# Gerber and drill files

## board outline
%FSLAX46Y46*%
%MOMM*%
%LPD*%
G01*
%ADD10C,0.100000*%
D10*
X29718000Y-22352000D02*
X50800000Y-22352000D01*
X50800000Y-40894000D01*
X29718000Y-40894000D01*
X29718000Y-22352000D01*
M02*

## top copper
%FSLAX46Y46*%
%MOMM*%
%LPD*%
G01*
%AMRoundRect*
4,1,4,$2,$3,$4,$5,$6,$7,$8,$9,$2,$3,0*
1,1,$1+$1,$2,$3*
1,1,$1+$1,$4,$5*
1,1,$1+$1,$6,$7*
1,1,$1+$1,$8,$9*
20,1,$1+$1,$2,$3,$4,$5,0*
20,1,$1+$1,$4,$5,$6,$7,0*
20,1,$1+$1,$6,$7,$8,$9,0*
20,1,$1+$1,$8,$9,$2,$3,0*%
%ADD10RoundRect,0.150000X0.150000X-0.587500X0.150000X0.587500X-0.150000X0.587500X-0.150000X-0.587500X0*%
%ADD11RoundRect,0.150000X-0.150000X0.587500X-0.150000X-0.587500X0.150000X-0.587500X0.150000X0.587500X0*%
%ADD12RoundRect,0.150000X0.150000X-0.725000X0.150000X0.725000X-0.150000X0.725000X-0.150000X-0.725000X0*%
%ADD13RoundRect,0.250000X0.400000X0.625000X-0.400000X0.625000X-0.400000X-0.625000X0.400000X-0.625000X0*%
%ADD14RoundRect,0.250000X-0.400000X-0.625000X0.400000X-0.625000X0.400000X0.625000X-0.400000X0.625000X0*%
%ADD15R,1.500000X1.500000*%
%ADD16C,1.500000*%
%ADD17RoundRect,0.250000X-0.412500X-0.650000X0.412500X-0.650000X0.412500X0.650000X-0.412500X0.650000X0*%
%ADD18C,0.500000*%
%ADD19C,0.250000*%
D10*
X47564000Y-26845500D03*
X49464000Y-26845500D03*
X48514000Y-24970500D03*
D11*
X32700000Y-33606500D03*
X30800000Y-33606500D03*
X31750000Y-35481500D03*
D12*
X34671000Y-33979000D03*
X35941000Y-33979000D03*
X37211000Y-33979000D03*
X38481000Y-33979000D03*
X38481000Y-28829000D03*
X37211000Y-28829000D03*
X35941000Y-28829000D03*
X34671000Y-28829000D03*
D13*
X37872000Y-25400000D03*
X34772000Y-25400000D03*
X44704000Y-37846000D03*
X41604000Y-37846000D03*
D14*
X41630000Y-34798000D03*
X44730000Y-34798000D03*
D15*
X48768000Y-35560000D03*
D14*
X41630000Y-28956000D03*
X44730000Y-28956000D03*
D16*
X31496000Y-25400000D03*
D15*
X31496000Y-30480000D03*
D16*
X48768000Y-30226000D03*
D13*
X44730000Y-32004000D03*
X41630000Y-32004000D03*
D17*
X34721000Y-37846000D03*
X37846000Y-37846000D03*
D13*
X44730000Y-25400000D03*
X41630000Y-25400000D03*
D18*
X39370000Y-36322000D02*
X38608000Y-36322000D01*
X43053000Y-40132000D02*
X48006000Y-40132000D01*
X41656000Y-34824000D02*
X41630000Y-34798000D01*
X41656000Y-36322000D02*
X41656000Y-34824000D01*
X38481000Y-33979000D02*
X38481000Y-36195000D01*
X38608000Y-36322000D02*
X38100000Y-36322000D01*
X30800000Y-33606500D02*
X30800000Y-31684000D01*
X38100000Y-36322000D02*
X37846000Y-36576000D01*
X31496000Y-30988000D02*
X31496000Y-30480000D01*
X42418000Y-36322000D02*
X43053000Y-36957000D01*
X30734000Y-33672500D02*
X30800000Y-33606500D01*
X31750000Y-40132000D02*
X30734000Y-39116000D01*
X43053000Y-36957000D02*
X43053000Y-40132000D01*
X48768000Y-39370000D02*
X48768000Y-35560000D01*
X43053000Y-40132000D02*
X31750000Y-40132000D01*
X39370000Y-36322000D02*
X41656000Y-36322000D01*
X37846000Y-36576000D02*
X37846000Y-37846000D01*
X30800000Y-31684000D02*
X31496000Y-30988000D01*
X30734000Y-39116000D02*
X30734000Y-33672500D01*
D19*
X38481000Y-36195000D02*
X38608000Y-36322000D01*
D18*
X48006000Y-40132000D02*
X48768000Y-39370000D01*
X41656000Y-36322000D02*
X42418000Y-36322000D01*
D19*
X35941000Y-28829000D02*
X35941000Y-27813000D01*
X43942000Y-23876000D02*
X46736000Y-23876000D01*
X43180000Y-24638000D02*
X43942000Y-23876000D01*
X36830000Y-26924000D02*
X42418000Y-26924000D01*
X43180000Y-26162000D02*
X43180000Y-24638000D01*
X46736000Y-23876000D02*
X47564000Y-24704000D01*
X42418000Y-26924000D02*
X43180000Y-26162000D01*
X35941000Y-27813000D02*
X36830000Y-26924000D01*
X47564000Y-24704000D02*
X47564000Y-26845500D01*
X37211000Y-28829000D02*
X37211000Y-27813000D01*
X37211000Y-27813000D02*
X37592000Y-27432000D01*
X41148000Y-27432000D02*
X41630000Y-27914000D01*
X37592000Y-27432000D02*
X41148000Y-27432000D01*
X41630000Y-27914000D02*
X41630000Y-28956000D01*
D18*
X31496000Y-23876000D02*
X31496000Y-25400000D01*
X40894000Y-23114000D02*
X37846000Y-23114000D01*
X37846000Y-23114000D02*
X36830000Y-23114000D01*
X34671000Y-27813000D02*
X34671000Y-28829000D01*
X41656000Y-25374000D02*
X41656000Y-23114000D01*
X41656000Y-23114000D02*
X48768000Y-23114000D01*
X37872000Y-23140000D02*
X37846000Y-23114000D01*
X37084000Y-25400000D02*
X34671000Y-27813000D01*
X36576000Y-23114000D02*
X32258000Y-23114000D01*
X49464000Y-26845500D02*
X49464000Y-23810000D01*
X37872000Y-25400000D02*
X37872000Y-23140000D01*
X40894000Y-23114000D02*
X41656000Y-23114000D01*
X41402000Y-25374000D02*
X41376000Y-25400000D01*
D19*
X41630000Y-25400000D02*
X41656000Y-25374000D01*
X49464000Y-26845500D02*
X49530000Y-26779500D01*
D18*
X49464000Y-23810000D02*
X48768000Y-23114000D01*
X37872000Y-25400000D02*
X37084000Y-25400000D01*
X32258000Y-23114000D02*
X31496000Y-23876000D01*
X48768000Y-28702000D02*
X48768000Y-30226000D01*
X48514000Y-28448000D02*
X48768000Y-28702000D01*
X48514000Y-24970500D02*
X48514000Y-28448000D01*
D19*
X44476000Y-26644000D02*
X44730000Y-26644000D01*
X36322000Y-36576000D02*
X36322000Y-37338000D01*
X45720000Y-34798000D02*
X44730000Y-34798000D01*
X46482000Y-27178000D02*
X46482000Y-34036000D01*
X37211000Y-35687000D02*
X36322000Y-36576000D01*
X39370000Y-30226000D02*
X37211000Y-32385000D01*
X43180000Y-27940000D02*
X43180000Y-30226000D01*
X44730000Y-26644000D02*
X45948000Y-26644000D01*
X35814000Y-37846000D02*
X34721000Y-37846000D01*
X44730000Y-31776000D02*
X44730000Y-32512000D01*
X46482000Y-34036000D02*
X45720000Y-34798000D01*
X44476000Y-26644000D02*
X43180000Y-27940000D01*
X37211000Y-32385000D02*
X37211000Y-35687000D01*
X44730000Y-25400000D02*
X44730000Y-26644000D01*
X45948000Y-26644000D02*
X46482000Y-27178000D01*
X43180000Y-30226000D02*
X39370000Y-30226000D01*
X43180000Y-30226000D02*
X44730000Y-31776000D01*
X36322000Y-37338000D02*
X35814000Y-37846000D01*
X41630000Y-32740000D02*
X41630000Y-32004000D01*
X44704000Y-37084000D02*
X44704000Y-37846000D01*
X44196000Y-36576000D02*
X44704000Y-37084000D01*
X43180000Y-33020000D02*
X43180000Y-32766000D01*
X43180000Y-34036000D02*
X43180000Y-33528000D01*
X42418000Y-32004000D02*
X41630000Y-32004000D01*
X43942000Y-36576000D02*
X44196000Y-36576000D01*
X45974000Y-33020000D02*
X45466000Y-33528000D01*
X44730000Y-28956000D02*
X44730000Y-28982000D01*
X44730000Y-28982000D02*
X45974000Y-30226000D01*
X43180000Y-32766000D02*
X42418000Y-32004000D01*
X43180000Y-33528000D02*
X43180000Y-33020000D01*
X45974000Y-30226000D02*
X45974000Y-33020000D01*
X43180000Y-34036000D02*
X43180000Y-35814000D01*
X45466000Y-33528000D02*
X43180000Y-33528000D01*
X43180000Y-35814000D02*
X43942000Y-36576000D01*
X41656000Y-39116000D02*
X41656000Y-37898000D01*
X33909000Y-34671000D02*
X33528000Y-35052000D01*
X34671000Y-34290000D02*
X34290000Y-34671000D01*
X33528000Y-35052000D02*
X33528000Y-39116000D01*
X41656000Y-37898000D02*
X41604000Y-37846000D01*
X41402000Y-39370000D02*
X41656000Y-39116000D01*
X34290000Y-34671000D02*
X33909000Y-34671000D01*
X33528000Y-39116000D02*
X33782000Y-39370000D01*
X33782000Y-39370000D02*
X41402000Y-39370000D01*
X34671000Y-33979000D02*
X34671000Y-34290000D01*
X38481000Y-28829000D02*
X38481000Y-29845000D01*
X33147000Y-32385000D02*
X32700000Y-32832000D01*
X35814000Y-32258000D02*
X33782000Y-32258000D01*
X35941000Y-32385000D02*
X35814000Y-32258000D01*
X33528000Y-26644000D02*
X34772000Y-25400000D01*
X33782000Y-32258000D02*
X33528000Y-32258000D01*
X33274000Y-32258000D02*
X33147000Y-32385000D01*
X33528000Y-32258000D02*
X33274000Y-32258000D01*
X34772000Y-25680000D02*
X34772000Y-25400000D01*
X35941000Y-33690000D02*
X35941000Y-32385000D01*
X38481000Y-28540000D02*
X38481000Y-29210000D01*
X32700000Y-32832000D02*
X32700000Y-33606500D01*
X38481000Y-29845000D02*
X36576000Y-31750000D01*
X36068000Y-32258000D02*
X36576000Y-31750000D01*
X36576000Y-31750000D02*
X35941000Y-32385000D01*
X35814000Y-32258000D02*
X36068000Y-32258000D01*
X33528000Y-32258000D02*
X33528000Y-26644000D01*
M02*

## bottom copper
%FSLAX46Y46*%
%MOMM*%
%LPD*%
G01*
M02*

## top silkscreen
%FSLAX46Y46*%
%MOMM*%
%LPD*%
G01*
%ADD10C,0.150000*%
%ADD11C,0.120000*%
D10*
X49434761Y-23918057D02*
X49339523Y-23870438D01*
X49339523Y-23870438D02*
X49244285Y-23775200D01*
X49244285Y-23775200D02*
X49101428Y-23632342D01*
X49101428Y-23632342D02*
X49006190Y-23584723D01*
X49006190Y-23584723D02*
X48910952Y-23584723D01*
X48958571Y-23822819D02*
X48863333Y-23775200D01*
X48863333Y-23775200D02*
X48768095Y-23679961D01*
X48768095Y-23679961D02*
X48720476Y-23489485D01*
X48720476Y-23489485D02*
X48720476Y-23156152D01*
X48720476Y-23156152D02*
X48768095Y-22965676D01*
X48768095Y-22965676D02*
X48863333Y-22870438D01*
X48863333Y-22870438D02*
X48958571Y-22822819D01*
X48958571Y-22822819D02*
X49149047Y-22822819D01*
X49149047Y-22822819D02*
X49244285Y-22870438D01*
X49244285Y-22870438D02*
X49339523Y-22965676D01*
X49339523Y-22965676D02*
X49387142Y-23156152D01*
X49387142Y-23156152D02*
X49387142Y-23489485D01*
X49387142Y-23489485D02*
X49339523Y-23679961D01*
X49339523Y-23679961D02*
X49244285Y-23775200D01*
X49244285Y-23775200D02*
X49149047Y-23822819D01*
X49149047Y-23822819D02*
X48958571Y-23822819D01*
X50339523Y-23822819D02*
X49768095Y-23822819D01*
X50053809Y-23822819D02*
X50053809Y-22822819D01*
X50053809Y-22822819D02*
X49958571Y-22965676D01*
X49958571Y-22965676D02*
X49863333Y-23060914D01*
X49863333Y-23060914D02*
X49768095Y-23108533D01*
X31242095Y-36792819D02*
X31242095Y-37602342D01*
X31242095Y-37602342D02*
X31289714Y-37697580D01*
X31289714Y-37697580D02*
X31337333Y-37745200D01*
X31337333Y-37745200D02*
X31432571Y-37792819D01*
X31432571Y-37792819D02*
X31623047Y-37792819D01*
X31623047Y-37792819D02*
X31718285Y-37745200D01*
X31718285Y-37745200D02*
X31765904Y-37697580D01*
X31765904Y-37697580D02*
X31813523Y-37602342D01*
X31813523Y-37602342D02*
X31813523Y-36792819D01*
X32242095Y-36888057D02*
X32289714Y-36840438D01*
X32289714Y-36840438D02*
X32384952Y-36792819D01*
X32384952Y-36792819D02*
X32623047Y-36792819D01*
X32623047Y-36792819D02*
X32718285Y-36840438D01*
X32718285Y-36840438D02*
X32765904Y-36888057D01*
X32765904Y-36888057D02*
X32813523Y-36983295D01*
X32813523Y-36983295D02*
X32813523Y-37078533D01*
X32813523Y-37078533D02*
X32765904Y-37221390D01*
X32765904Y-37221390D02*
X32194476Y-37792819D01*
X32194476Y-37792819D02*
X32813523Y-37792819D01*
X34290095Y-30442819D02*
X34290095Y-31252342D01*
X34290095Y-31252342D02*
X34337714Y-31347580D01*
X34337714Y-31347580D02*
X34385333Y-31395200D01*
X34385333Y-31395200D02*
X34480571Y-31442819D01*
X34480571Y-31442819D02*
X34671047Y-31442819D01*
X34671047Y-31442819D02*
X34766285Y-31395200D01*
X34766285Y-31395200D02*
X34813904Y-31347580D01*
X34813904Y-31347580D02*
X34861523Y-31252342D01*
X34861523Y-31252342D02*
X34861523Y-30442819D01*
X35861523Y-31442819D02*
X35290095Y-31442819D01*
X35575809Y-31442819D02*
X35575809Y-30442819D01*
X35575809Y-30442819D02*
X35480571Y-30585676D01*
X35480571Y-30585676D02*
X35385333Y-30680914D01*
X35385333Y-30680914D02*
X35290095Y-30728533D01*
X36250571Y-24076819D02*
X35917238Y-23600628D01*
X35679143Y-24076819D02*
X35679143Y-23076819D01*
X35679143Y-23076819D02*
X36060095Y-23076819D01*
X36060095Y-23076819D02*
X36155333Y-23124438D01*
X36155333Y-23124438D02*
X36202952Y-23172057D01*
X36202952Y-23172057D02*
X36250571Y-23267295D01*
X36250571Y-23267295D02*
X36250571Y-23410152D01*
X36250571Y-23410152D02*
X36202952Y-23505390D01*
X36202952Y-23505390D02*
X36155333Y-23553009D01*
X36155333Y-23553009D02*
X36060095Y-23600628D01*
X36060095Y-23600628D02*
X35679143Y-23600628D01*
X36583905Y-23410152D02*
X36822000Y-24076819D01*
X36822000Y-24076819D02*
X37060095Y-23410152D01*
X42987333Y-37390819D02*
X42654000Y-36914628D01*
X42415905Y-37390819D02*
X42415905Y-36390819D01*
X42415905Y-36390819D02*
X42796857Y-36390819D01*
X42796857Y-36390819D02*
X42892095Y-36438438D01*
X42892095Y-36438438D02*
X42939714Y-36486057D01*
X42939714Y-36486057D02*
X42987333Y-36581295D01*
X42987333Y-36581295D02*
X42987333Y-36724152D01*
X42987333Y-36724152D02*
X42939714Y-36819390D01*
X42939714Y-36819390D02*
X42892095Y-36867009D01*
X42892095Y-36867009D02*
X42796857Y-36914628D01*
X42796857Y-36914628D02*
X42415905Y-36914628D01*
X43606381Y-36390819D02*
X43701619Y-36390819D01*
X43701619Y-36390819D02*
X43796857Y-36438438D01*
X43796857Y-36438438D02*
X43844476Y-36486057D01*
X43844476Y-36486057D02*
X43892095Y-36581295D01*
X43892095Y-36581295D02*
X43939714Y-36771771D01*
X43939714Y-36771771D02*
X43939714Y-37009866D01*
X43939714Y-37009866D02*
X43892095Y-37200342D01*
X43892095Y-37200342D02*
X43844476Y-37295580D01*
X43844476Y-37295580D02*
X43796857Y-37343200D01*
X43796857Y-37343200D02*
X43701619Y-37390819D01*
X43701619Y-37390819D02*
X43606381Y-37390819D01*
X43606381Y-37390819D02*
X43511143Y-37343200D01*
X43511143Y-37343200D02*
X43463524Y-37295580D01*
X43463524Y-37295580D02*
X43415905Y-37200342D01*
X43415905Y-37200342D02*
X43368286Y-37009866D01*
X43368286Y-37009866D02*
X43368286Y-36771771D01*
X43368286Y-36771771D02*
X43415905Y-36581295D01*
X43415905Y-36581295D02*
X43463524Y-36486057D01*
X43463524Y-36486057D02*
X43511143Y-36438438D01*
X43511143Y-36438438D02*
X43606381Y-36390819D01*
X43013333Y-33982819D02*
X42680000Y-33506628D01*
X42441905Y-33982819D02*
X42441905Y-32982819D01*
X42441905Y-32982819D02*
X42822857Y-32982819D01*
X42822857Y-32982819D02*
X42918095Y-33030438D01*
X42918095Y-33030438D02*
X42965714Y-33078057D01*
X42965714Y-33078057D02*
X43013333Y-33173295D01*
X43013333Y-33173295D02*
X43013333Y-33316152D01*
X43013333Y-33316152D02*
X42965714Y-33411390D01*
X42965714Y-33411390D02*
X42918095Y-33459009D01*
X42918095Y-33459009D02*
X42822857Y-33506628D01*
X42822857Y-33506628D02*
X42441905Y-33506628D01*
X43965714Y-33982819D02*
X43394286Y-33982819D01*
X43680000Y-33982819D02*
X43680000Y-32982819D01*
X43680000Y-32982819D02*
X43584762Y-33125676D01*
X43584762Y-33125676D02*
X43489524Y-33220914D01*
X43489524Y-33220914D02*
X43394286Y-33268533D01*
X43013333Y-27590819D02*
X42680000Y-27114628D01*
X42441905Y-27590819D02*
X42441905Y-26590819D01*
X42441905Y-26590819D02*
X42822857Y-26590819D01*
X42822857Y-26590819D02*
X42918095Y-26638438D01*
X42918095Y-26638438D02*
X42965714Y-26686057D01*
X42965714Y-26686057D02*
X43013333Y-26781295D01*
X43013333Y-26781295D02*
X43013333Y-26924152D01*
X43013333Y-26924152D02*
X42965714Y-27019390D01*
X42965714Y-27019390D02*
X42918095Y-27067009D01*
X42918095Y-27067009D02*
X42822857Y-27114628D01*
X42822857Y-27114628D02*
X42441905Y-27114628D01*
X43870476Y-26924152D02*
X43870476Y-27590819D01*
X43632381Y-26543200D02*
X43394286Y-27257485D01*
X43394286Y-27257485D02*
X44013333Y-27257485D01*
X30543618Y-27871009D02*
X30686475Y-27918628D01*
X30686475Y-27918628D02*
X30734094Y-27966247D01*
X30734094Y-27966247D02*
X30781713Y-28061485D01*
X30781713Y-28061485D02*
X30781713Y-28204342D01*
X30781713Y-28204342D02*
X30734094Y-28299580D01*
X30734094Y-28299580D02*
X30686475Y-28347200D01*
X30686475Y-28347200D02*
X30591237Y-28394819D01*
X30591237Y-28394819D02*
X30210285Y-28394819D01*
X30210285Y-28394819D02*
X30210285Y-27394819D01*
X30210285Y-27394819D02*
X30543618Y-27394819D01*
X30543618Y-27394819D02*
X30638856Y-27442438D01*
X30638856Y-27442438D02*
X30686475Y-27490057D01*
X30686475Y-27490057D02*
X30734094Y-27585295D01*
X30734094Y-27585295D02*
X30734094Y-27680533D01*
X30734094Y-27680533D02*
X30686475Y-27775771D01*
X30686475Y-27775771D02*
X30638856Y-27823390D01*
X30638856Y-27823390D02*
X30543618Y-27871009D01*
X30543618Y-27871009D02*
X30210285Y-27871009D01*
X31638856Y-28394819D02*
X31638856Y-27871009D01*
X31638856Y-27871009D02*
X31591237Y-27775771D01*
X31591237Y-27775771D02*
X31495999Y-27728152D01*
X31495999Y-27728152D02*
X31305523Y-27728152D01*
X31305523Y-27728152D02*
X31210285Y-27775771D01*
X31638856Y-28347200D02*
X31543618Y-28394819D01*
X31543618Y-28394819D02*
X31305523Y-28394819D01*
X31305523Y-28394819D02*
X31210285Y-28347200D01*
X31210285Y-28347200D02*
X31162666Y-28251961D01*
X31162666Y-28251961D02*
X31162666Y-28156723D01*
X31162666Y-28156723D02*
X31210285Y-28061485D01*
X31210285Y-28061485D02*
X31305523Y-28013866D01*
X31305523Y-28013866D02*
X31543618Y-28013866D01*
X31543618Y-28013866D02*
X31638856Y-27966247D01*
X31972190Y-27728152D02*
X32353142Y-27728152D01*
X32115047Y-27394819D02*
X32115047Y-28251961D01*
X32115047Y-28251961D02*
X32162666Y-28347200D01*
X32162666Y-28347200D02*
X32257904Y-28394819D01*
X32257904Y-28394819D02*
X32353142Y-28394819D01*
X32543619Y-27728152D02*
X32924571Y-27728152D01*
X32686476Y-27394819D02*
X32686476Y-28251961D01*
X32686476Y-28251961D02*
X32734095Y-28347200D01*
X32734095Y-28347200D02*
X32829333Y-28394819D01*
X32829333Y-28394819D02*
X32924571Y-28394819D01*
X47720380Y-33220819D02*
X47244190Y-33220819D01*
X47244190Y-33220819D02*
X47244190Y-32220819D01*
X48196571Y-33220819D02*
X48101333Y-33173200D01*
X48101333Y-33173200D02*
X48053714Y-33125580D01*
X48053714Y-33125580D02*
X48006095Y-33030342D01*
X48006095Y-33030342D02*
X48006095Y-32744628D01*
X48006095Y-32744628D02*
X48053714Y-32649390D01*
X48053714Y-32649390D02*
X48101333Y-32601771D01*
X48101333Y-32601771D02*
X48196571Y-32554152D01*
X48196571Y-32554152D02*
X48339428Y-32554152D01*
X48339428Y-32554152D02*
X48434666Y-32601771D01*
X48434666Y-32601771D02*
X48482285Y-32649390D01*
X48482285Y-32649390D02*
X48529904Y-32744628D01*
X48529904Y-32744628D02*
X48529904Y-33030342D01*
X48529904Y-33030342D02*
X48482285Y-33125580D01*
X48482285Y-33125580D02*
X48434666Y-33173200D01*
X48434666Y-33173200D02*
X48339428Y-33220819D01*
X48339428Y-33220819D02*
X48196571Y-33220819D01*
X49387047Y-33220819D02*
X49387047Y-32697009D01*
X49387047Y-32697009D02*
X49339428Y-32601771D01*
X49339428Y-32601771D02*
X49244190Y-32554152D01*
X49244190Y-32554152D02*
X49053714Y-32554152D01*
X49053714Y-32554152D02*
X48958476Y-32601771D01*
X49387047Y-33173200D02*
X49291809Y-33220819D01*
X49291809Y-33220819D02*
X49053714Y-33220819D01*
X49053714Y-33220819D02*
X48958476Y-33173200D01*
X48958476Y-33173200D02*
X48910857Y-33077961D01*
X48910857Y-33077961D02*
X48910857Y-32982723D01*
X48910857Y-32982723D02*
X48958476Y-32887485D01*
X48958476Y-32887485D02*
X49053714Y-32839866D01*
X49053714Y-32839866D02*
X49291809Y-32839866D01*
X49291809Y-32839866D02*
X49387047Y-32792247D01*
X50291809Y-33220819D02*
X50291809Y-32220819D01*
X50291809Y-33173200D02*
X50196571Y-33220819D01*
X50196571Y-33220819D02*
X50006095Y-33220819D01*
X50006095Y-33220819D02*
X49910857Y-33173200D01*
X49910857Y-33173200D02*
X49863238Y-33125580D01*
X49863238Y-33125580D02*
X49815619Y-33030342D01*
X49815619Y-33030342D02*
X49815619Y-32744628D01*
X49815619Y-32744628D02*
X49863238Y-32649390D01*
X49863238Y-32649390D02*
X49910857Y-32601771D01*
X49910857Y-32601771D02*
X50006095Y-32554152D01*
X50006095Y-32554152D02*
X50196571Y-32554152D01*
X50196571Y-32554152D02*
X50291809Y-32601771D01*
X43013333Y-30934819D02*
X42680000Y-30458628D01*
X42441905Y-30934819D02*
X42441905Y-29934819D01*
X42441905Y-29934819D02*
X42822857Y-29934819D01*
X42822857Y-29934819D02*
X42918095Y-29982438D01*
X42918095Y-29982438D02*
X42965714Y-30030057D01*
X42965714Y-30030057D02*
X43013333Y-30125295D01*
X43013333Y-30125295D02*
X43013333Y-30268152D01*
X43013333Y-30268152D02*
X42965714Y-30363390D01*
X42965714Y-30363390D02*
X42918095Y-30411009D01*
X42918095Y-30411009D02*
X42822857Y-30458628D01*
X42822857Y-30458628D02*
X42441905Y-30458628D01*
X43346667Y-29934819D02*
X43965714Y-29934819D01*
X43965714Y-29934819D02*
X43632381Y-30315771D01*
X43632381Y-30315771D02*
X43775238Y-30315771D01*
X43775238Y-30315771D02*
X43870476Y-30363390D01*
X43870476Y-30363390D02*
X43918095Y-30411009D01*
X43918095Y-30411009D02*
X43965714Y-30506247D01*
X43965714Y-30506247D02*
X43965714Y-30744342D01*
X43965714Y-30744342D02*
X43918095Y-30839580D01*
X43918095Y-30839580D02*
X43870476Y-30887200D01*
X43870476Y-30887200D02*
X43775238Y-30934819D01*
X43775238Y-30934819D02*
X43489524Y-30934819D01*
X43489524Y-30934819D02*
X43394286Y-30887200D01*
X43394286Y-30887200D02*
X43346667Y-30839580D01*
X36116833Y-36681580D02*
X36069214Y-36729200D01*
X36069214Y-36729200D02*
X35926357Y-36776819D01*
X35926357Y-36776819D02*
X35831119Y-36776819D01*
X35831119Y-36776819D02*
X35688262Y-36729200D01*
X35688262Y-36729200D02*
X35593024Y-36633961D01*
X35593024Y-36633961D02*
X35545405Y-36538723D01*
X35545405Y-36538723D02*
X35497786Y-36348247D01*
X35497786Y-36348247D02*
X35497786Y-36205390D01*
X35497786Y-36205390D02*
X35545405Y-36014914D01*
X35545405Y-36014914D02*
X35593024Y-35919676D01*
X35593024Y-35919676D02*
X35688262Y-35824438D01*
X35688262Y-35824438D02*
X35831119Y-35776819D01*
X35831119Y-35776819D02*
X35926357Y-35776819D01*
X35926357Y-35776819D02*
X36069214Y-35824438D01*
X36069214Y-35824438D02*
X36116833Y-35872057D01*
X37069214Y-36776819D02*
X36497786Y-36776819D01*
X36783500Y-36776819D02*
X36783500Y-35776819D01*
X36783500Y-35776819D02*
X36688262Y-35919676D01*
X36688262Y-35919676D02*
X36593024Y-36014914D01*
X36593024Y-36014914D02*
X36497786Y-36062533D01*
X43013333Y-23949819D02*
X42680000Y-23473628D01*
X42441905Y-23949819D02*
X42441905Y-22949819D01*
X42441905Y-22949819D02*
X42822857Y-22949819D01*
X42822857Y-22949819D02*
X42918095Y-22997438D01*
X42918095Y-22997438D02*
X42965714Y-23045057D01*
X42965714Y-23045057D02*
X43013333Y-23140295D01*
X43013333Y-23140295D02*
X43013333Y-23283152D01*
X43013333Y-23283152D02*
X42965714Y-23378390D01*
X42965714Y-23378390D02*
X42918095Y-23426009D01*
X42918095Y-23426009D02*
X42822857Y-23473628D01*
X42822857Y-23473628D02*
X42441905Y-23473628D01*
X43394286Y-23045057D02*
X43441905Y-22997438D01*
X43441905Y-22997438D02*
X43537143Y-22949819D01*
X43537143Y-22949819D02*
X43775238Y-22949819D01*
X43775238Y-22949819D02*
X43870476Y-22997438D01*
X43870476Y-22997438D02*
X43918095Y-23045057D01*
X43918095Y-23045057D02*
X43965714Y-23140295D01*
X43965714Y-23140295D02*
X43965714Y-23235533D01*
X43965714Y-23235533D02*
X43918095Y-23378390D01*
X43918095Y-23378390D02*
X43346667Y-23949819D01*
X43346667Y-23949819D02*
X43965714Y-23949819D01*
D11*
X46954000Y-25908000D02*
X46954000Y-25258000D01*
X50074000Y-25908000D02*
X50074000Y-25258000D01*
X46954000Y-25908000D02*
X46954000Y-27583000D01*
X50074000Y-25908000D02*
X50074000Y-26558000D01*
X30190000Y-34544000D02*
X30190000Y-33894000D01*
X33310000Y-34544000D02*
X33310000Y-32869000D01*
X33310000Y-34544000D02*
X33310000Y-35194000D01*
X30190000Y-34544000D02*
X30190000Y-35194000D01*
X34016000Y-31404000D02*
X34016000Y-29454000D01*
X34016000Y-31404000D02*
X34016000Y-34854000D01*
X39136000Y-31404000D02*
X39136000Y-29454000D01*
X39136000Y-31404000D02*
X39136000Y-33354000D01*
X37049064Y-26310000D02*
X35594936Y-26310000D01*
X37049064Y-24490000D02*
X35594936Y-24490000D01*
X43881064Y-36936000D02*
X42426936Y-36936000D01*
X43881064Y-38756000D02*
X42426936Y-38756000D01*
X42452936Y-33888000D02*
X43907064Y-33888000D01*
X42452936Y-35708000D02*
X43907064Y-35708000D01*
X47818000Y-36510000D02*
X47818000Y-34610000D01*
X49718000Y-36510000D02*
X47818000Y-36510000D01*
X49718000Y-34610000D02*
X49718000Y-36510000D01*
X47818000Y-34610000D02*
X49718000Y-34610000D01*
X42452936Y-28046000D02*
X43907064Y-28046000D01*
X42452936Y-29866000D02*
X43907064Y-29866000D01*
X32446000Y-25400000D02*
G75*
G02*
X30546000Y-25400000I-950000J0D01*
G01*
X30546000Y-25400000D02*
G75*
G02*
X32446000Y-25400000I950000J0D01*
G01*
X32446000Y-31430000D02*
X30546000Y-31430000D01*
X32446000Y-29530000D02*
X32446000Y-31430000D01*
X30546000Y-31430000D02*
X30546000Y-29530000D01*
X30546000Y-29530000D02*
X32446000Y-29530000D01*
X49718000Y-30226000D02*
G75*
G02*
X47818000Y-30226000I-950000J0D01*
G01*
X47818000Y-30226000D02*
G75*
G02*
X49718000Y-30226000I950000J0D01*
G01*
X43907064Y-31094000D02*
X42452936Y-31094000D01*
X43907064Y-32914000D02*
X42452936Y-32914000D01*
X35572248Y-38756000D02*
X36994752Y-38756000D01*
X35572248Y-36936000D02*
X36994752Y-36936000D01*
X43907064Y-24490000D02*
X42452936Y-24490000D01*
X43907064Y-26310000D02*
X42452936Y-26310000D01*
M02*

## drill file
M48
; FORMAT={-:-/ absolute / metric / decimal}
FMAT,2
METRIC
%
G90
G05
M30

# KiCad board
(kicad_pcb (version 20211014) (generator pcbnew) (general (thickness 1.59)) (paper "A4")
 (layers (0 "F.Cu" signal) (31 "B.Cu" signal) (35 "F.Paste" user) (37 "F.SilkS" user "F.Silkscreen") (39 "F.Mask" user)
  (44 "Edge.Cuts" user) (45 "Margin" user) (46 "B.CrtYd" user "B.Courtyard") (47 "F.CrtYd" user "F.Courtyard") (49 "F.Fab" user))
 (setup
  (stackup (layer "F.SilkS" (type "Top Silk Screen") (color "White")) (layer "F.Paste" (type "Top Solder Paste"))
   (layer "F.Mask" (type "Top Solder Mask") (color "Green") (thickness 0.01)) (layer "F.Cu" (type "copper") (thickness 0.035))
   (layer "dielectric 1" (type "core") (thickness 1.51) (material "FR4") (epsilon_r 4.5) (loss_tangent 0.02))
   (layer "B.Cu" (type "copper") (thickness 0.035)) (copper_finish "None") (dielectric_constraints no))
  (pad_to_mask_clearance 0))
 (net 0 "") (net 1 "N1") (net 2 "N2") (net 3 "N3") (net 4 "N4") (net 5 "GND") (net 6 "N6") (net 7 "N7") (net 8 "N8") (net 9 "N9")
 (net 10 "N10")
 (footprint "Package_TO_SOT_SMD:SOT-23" (layer "F.Cu") (at 48.514 25.908 90)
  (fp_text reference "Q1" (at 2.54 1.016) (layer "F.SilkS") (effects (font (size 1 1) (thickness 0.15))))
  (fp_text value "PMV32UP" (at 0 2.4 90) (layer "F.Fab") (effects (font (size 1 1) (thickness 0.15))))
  (fp_line (start 0 -1.56) (end 0.65 -1.56) (layer "F.SilkS") (width 0.12))
  (fp_line (start 0 1.56) (end 0.65 1.56) (layer "F.SilkS") (width 0.12))
  (fp_line (start 0 -1.56) (end -1.675 -1.56) (layer "F.SilkS") (width 0.12))
  (fp_line (start 0 1.56) (end -0.65 1.56) (layer "F.SilkS") (width 0.12))
  (pad "1" smd roundrect (at -0.9375 -0.95 90) (size 1.475 0.6) (layers "F.Cu" "F.Paste" "F.Mask") (roundrect_rratio 0.25) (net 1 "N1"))
  (pad "2" smd roundrect (at -0.9375 0.95 90) (size 1.475 0.6) (layers "F.Cu" "F.Paste" "F.Mask") (roundrect_rratio 0.25) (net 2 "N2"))
  (pad "3" smd roundrect (at 0.9375 0 90) (size 1.475 0.6) (layers "F.Cu" "F.Paste" "F.Mask") (roundrect_rratio 0.25) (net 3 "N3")))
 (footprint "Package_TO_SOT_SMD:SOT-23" (layer "F.Cu") (at 31.75 34.544 -90)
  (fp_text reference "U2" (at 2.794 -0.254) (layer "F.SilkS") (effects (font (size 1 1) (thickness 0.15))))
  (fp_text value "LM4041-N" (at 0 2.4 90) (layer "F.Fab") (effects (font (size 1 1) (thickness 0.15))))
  (fp_line (start 0 1.56) (end -0.65 1.56) (layer "F.SilkS") (width 0.12))
  (fp_line (start 0 -1.56) (end -1.675 -1.56) (layer "F.SilkS") (width 0.12))
  (fp_line (start 0 -1.56) (end 0.65 -1.56) (layer "F.SilkS") (width 0.12))
  (fp_line (start 0 1.56) (end 0.65 1.56) (layer "F.SilkS") (width 0.12))
  (pad "1" smd roundrect (at -0.9375 -0.95 270) (size 1.475 0.6) (layers "F.Cu" "F.Paste" "F.Mask") (roundrect_rratio 0.25) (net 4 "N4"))
  (pad "2" smd roundrect (at -0.9375 0.95 270) (size 1.475 0.6) (layers "F.Cu" "F.Paste" "F.Mask") (roundrect_rratio 0.25) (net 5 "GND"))
  (pad "3" smd roundrect (at 0.9375 0 270) (size 1.475 0.6) (layers "F.Cu" "F.Paste" "F.Mask") (roundrect_rratio 0.25) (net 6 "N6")))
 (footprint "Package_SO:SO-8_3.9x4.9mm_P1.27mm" (layer "F.Cu") (at 36.576 31.404 90)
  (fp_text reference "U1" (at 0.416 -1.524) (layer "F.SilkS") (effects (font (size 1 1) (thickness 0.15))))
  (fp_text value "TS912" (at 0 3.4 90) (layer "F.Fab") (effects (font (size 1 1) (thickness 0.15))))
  (fp_line (start 0 -2.56) (end 1.95 -2.56) (layer "F.SilkS") (width 0.12))
  (fp_line (start 0 -2.56) (end -3.45 -2.56) (layer "F.SilkS") (width 0.12))
  (fp_line (start 0 2.56) (end 1.95 2.56) (layer "F.SilkS") (width 0.12))
  (fp_line (start 0 2.56) (end -1.95 2.56) (layer "F.SilkS") (width 0.12))
  (pad "1" smd roundrect (at -2.575 -1.905 90) (size 1.75 0.6) (layers "F.Cu" "F.Paste" "F.Mask") (roundrect_rratio 0.25) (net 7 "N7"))
  (pad "2" smd roundrect (at -2.575 -0.635 90) (size 1.75 0.6) (layers "F.Cu" "F.Paste" "F.Mask") (roundrect_rratio 0.25) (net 4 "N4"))
  (pad "3" smd roundrect (at -2.575 0.635 90) (size 1.75 0.6) (layers "F.Cu" "F.Paste" "F.Mask") (roundrect_rratio 0.25) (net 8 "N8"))
  (pad "4" smd roundrect (at -2.575 1.905 90) (size 1.75 0.6) (layers "F.Cu" "F.Paste" "F.Mask") (roundrect_rratio 0.25) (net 5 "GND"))
  (pad "5" smd roundrect (at 2.575 1.905 90) (size 1.75 0.6) (layers "F.Cu" "F.Paste" "F.Mask") (roundrect_rratio 0.25) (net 4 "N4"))
  (pad "6" smd roundrect (at 2.575 0.635 90) (size 1.75 0.6) (layers "F.Cu" "F.Paste" "F.Mask") (roundrect_rratio 0.25) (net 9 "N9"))
  (pad "7" smd roundrect (at 2.575 -0.635 90) (size 1.75 0.6) (layers "F.Cu" "F.Paste" "F.Mask") (roundrect_rratio 0.25) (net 1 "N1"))
  (pad "8" smd roundrect (at 2.575 -1.905 90) (size 1.75 0.6) (layers "F.Cu" "F.Paste" "F.Mask") (roundrect_rratio 0.25) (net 2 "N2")))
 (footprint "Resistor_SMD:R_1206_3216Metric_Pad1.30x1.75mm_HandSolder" (layer "F.Cu") (at 36.322 25.4 180)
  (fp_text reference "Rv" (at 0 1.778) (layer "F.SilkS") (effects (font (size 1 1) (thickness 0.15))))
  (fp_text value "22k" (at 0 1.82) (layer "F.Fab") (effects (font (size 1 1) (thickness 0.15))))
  (fp_line (start -0.727064 -0.91) (end 0.727064 -0.91) (layer "F.SilkS") (width 0.12))
  (fp_line (start -0.727064 0.91) (end 0.727064 0.91) (layer "F.SilkS") (width 0.12))
  (pad "1" smd roundrect (at -1.55 0 180) (size 1.3 1.75) (layers "F.Cu" "F.Paste" "F.Mask") (roundrect_rratio 0.1923076923) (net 2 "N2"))
  (pad "2" smd roundrect (at 1.55 0 180) (size 1.3 1.75) (layers "F.Cu" "F.Paste" "F.Mask") (roundrect_rratio 0.1923076923) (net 4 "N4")))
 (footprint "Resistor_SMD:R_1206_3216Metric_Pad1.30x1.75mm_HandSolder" (layer "F.Cu") (at 43.154 37.846 180)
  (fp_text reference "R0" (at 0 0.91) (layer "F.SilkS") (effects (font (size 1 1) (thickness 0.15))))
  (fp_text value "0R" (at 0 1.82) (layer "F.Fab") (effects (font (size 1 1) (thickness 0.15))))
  (fp_line (start -0.727064 0.91) (end 0.727064 0.91) (layer "F.SilkS") (width 0.12))
  (fp_line (start -0.727064 -0.91) (end 0.727064 -0.91) (layer "F.SilkS") (width 0.12))
  (pad "1" smd roundrect (at -1.55 0 180) (size 1.3 1.75) (layers "F.Cu" "F.Paste" "F.Mask") (roundrect_rratio 0.192308) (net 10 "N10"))
  (pad "2" smd roundrect (at 1.55 0 180) (size 1.3 1.75) (layers "F.Cu" "F.Paste" "F.Mask") (roundrect_rratio 0.192308) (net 7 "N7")))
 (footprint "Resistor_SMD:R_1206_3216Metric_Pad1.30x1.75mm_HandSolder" (layer "F.Cu") (at 43.18 34.798)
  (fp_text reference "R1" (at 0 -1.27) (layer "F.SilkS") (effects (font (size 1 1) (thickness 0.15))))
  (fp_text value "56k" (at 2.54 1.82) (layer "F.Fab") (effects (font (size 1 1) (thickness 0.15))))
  (fp_line (start -0.727064 -0.91) (end 0.727064 -0.91) (layer "F.SilkS") (width 0.12))
  (fp_line (start -0.727064 0.91) (end 0.727064 0.91) (layer "F.SilkS") (width 0.12))
  (pad "1" smd roundrect (at -1.55 0) (size 1.3 1.75) (layers "F.Cu" "F.Paste" "F.Mask") (roundrect_rratio 0.1923076923) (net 5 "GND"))
  (pad "2" smd roundrect (at 1.55 0) (size 1.3 1.75) (layers "F.Cu" "F.Paste" "F.Mask") (roundrect_rratio 0.1923076923) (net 8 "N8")))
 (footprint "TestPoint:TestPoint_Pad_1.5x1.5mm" (layer "F.Cu") (at 48.768 35.56)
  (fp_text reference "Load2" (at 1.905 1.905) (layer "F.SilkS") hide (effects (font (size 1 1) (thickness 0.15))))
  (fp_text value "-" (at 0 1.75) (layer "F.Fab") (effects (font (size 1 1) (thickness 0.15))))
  (fp_line (start -0.95 0.95) (end -0.95 -0.95) (layer "F.SilkS") (width 0.12))
  (fp_line (start 0.95 0.95) (end -0.95 0.95) (layer "F.SilkS") (width 0.12))
  (fp_line (start 0.95 -0.95) (end 0.95 0.95) (layer "F.SilkS") (width 0.12))
  (fp_line (start -0.95 -0.95) (end 0.95 -0.95) (layer "F.SilkS") (width 0.12))
  (pad "1" smd rect (at 0 0) (size 1.5 1.5) (layers "F.Cu" "F.Mask") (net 5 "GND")))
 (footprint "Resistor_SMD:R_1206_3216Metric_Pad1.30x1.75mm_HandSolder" (layer "F.Cu") (at 43.18 28.956)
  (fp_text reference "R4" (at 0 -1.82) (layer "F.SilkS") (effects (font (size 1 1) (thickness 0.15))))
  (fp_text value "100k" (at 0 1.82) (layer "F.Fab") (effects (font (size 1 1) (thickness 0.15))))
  (fp_line (start -0.727064 -0.91) (end 0.727064 -0.91) (layer "F.SilkS") (width 0.12))
  (fp_line (start -0.727064 0.91) (end 0.727064 0.91) (layer "F.SilkS") (width 0.12))
  (pad "1" smd roundrect (at -1.55 0) (size 1.3 1.75) (layers "F.Cu" "F.Paste" "F.Mask") (roundrect_rratio 0.1923076923) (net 9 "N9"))
  (pad "2" smd roundrect (at 1.55 0) (size 1.3 1.75) (layers "F.Cu" "F.Paste" "F.Mask") (roundrect_rratio 0.1923076923) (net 10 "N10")))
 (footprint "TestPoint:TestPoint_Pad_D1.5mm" (layer "F.Cu") (at 31.496 25.4)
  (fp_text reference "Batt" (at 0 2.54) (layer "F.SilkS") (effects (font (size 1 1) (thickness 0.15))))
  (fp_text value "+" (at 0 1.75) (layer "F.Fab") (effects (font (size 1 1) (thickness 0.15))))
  (fp_circle (center 0 0) (end 0 0.95) (layer "F.SilkS") (width 0.12) (fill none))
  (pad "1" smd circle (at 0 0) (size 1.5 1.5) (layers "F.Cu" "F.Mask") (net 2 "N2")))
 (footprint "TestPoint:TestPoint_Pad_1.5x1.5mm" (layer "F.Cu") (at 31.496 30.48)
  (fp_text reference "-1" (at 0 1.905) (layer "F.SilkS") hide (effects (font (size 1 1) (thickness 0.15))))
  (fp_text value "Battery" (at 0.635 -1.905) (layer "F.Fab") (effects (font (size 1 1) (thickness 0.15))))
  (fp_line (start 0.95 0.95) (end -0.95 0.95) (layer "F.SilkS") (width 0.12))
  (fp_line (start 0.95 -0.95) (end 0.95 0.95) (layer "F.SilkS") (width 0.12))
  (fp_line (start -0.95 0.95) (end -0.95 -0.95) (layer "F.SilkS") (width 0.12))
  (fp_line (start -0.95 -0.95) (end 0.95 -0.95) (layer "F.SilkS") (width 0.12))
  (pad "1" smd rect (at 0 0) (size 1.5 1.5) (layers "F.Cu" "F.Mask") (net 5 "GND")))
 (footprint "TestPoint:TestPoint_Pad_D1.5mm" (layer "F.Cu") (at 48.768 30.226)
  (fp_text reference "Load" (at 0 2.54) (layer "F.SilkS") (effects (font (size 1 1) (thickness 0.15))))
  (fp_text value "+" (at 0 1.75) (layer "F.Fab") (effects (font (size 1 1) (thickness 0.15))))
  (fp_circle (center 0 0) (end 0 0.95) (layer "F.SilkS") (width 0.12) (fill none))
  (pad "1" smd circle (at 0 0) (size 1.5 1.5) (layers "F.Cu" "F.Mask") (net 3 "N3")))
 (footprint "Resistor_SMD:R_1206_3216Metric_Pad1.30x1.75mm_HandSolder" (layer "F.Cu") (at 43.18 32.004 180)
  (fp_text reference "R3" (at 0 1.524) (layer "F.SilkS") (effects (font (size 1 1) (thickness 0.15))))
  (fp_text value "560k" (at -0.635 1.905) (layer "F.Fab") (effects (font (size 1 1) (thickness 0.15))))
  (fp_line (start -0.727064 0.91) (end 0.727064 0.91) (layer "F.SilkS") (width 0.12))
  (fp_line (start -0.727064 -0.91) (end 0.727064 -0.91) (layer "F.SilkS") (width 0.12))
  (pad "1" smd roundrect (at -1.55 0 180) (size 1.3 1.75) (layers "F.Cu" "F.Paste" "F.Mask") (roundrect_rratio 0.1923076923) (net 8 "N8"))
  (pad "2" smd roundrect (at 1.55 0 180) (size 1.3 1.75) (layers "F.Cu" "F.Paste" "F.Mask") (roundrect_rratio 0.1923076923) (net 10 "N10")))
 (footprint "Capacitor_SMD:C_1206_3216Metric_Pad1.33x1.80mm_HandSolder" (layer "F.Cu") (at 36.2835 37.846)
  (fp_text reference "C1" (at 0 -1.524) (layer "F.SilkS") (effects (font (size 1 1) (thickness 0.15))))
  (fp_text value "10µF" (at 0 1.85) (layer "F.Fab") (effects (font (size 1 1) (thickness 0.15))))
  (fp_line (start -0.711252 0.91) (end 0.711252 0.91) (layer "F.SilkS") (width 0.12))
  (fp_line (start -0.711252 -0.91) (end 0.711252 -0.91) (layer "F.SilkS") (width 0.12))
  (pad "1" smd roundrect (at -1.5625 0) (size 1.325 1.8) (layers "F.Cu" "F.Paste" "F.Mask") (roundrect_rratio 0.1886792453) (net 8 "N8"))
  (pad "2" smd roundrect (at 1.5625 0) (size 1.325 1.8) (layers "F.Cu" "F.Paste" "F.Mask") (roundrect_rratio 0.1886792453) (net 5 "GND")))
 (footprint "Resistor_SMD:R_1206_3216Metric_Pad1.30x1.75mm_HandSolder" (layer "F.Cu") (at 43.18 25.4 180)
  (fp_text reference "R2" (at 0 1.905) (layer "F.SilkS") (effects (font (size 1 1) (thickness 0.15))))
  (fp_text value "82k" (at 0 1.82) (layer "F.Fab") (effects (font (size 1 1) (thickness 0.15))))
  (fp_line (start -0.727064 0.91) (end 0.727064 0.91) (layer "F.SilkS") (width 0.12))
  (fp_line (start -0.727064 -0.91) (end 0.727064 -0.91) (layer "F.SilkS") (width 0.12))
  (pad "1" smd roundrect (at -1.55 0 180) (size 1.3 1.75) (layers "F.Cu" "F.Paste" "F.Mask") (roundrect_rratio 0.1923076923) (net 8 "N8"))
  (pad "2" smd roundrect (at 1.55 0 180) (size 1.3 1.75) (layers "F.Cu" "F.Paste" "F.Mask") (roundrect_rratio 0.1923076923) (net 2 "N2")))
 (gr_rect (start 29.718 22.352) (end 50.8 40.894) (layer "Edge.Cuts") (width 0.1) (fill none))
 (segment (start 39.37 36.322) (end 38.608 36.322) (width 0.5) (layer "F.Cu") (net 5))
 (segment (start 43.053 40.132) (end 48.006 40.132) (width 0.5) (layer "F.Cu") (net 5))
 (segment (start 41.656 34.824) (end 41.63 34.798) (width 0.5) (layer "F.Cu") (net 5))
 (segment (start 41.656 36.322) (end 41.656 34.824) (width 0.5) (layer "F.Cu") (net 5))
 (segment (start 38.481 33.979) (end 38.481 36.195) (width 0.5) (layer "F.Cu") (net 5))
 (segment (start 38.608 36.322) (end 38.1 36.322) (width 0.5) (layer "F.Cu") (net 5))
 (segment (start 30.8 33.6065) (end 30.8 31.684) (width 0.5) (layer "F.Cu") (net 5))
 (segment (start 38.1 36.322) (end 37.846 36.576) (width 0.5) (layer "F.Cu") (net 5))
 (segment (start 31.496 30.988) (end 31.496 30.48) (width 0.5) (layer "F.Cu") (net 5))
 (segment (start 42.418 36.322) (end 43.053 36.957) (width 0.5) (layer "F.Cu") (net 5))
 (segment (start 30.734 33.6725) (end 30.8 33.6065) (width 0.5) (layer "F.Cu") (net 5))
 (segment (start 31.75 40.132) (end 30.734 39.116) (width 0.5) (layer "F.Cu") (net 5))
 (segment (start 43.053 36.957) (end 43.053 40.132) (width 0.5) (layer "F.Cu") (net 5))
 (segment (start 48.768 39.37) (end 48.768 35.56) (width 0.5) (layer "F.Cu") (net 5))
 (segment (start 43.053 40.132) (end 31.75 40.132) (width 0.5) (layer "F.Cu") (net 5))
 (segment (start 39.37 36.322) (end 41.656 36.322) (width 0.5) (layer "F.Cu") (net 5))
 (segment (start 37.846 36.576) (end 37.846 37.846) (width 0.5) (layer "F.Cu") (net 5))
 (segment (start 30.8 31.684) (end 31.496 30.988) (width 0.5) (layer "F.Cu") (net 5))
 (segment (start 30.734 39.116) (end 30.734 33.6725) (width 0.5) (layer "F.Cu") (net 5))
 (segment (start 38.481 36.195) (end 38.608 36.322) (width 0.25) (layer "F.Cu") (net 5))
 (segment (start 48.006 40.132) (end 48.768 39.37) (width 0.5) (layer "F.Cu") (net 5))
 (segment (start 41.656 36.322) (end 42.418 36.322) (width 0.5) (layer "F.Cu") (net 5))
 (segment (start 35.941 28.829) (end 35.941 27.813) (width 0.25) (layer "F.Cu") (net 1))
 (segment (start 43.942 23.876) (end 46.736 23.876) (width 0.25) (layer "F.Cu") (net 1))
 (segment (start 43.18 24.638) (end 43.942 23.876) (width 0.25) (layer "F.Cu") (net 1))
 (segment (start 36.83 26.924) (end 42.418 26.924) (width 0.25) (layer "F.Cu") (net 1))
 (segment (start 43.18 26.162) (end 43.18 24.638) (width 0.25) (layer "F.Cu") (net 1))
 (segment (start 46.736 23.876) (end 47.564 24.704) (width 0.25) (layer "F.Cu") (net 1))
 (segment (start 42.418 26.924) (end 43.18 26.162) (width 0.25) (layer "F.Cu") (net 1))
 (segment (start 35.941 27.813) (end 36.83 26.924) (width 0.25) (layer "F.Cu") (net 1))
 (segment (start 47.564 24.704) (end 47.564 26.8455) (width 0.25) (layer "F.Cu") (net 1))
 (segment (start 37.211 28.829) (end 37.211 27.813) (width 0.25) (layer "F.Cu") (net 9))
 (segment (start 37.211 27.813) (end 37.592 27.432) (width 0.25) (layer "F.Cu") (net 9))
 (segment (start 41.148 27.432) (end 41.63 27.914) (width 0.25) (layer "F.Cu") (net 9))
 (segment (start 37.592 27.432) (end 41.148 27.432) (width 0.25) (layer "F.Cu") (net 9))
 (segment (start 41.63 27.914) (end 41.63 28.956) (width 0.25) (layer "F.Cu") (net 9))
 (segment (start 31.496 23.876) (end 31.496 25.4) (width 0.5) (layer "F.Cu") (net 2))
 (segment (start 40.894 23.114) (end 37.846 23.114) (width 0.5) (layer "F.Cu") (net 2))
 (segment (start 37.846 23.114) (end 36.83 23.114) (width 0.5) (layer "F.Cu") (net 2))
 (segment (start 34.671 27.813) (end 34.671 28.829) (width 0.5) (layer "F.Cu") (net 2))
 (segment (start 41.656 25.374) (end 41.656 23.114) (width 0.5) (layer "F.Cu") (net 2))
 (segment (start 41.656 23.114) (end 48.768 23.114) (width 0.5) (layer "F.Cu") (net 2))
 (segment (start 37.872 23.14) (end 37.846 23.114) (width 0.5) (layer "F.Cu") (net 2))
 (segment (start 37.084 25.4) (end 34.671 27.813) (width 0.5) (layer "F.Cu") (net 2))
 (segment (start 36.576 23.114) (end 32.258 23.114) (width 0.5) (layer "F.Cu") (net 2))
 (segment (start 49.464 26.8455) (end 49.464 23.81) (width 0.5) (layer "F.Cu") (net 2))
 (segment (start 37.872 25.4) (end 37.872 23.14) (width 0.5) (layer "F.Cu") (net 2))
 (segment (start 40.894 23.114) (end 41.656 23.114) (width 0.5) (layer "F.Cu") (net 2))
 (segment (start 41.402 25.374) (end 41.376 25.4) (width 0.5) (layer "F.Cu") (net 2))
 (segment (start 41.63 25.4) (end 41.656 25.374) (width 0.25) (layer "F.Cu") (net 2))
 (segment (start 49.464 26.8455) (end 49.53 26.7795) (width 0.25) (layer "F.Cu") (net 2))
 (segment (start 49.464 23.81) (end 48.768 23.114) (width 0.5) (layer "F.Cu") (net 2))
 (segment (start 37.872 25.4) (end 37.084 25.4) (width 0.5) (layer "F.Cu") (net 2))
 (segment (start 32.258 23.114) (end 31.496 23.876) (width 0.5) (layer "F.Cu") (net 2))
 (segment (start 48.768 28.702) (end 48.768 30.226) (width 0.5) (layer "F.Cu") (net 3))
 (segment (start 48.514 28.448) (end 48.768 28.702) (width 0.5) (layer "F.Cu") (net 3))
 (segment (start 48.514 24.9705) (end 48.514 28.448) (width 0.5) (layer "F.Cu") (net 3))
 (segment (start 44.476 26.644) (end 44.73 26.644) (width 0.25) (layer "F.Cu") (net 8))
 (segment (start 36.322 36.576) (end 36.322 37.338) (width 0.25) (layer "F.Cu") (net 8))
 (segment (start 45.72 34.798) (end 44.73 34.798) (width 0.25) (layer "F.Cu") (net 8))
 (segment (start 46.482 27.178) (end 46.482 34.036) (width 0.25) (layer "F.Cu") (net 8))
 (segment (start 37.211 35.687) (end 36.322 36.576) (width 0.25) (layer "F.Cu") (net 8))
 (segment (start 39.37 30.226) (end 37.211 32.385) (width 0.25) (layer "F.Cu") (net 8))
 (segment (start 43.18 27.94) (end 43.18 30.226) (width 0.25) (layer "F.Cu") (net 8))
 (segment (start 44.73 26.644) (end 45.948 26.644) (width 0.25) (layer "F.Cu") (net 8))
 (segment (start 35.814 37.846) (end 34.721 37.846) (width 0.25) (layer "F.Cu") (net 8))
 (segment (start 44.73 31.776) (end 44.73 32.512) (width 0.25) (layer "F.Cu") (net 8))
 (segment (start 46.482 34.036) (end 45.72 34.798) (width 0.25) (layer "F.Cu") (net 8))
 (segment (start 44.476 26.644) (end 43.18 27.94) (width 0.25) (layer "F.Cu") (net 8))
 (segment (start 37.211 32.385) (end 37.211 35.687) (width 0.25) (layer "F.Cu") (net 8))
 (segment (start 44.73 25.4) (end 44.73 26.644) (width 0.25) (layer "F.Cu") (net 8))
 (segment (start 45.948 26.644) (end 46.482 27.178) (width 0.25) (layer "F.Cu") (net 8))
 (segment (start 43.18 30.226) (end 39.37 30.226) (width 0.25) (layer "F.Cu") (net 8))
 (segment (start 43.18 30.226) (end 44.73 31.776) (width 0.25) (layer "F.Cu") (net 8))
 (segment (start 36.322 37.338) (end 35.814 37.846) (width 0.25) (layer "F.Cu") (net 8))
 (segment (start 41.63 32.74) (end 41.63 32.004) (width 0.25) (layer "F.Cu") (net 10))
 (segment (start 44.704 37.084) (end 44.704 37.846) (width 0.25) (layer "F.Cu") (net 10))
 (segment (start 44.196 36.576) (end 44.704 37.084) (width 0.25) (layer "F.Cu") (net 10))
 (segment (start 43.18 33.02) (end 43.18 32.766) (width 0.25) (layer "F.Cu") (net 10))
 (segment (start 43.18 34.036) (end 43.18 33.528) (width 0.25) (layer "F.Cu") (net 10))
 (segment (start 42.418 32.004) (end 41.63 32.004) (width 0.25) (layer "F.Cu") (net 10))
 (segment (start 43.942 36.576) (end 44.196 36.576) (width 0.25) (layer "F.Cu") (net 10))
 (segment (start 45.974 33.02) (end 45.466 33.528) (width 0.25) (layer "F.Cu") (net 10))
 (segment (start 44.73 28.956) (end 44.73 28.982) (width 0.25) (layer "F.Cu") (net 10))
 (segment (start 44.73 28.982) (end 45.974 30.226) (width 0.25) (layer "F.Cu") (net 10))
 (segment (start 43.18 32.766) (end 42.418 32.004) (width 0.25) (layer "F.Cu") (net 10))
 (segment (start 43.18 33.528) (end 43.18 33.02) (width 0.25) (layer "F.Cu") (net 10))
 (segment (start 45.974 30.226) (end 45.974 33.02) (width 0.25) (layer "F.Cu") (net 10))
 (segment (start 43.18 34.036) (end 43.18 35.814) (width 0.25) (layer "F.Cu") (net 10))
 (segment (start 45.466 33.528) (end 43.18 33.528) (width 0.25) (layer "F.Cu") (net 10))
 (segment (start 43.18 35.814) (end 43.942 36.576) (width 0.25) (layer "F.Cu") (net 10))
 (segment (start 41.656 39.116) (end 41.656 37.898) (width 0.25) (layer "F.Cu") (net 7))
 (segment (start 33.909 34.671) (end 33.528 35.052) (width 0.25) (layer "F.Cu") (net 7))
 (segment (start 34.671 34.29) (end 34.29 34.671) (width 0.25) (layer "F.Cu") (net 7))
 (segment (start 33.528 35.052) (end 33.528 39.116) (width 0.25) (layer "F.Cu") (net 7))
 (segment (start 41.656 37.898) (end 41.604 37.846) (width 0.25) (layer "F.Cu") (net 7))
 (segment (start 41.402 39.37) (end 41.656 39.116) (width 0.25) (layer "F.Cu") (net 7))
 (segment (start 34.29 34.671) (end 33.909 34.671) (width 0.25) (layer "F.Cu") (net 7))
 (segment (start 33.528 39.116) (end 33.782 39.37) (width 0.25) (layer "F.Cu") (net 7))
 (segment (start 33.782 39.37) (end 41.402 39.37) (width 0.25) (layer "F.Cu") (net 7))
 (segment (start 34.671 33.979) (end 34.671 34.29) (width 0.25) (layer "F.Cu") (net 7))
 (segment (start 38.481 28.829) (end 38.481 29.845) (width 0.25) (layer "F.Cu") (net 4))
 (segment (start 33.147 32.385) (end 32.7 32.832) (width 0.25) (layer "F.Cu") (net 4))
 (segment (start 35.814 32.258) (end 33.782 32.258) (width 0.25) (layer "F.Cu") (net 4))
 (segment (start 35.941 32.385) (end 35.814 32.258) (width 0.25) (layer "F.Cu") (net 4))
 (segment (start 33.528 26.644) (end 34.772 25.4) (width 0.25) (layer "F.Cu") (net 4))
 (segment (start 33.782 32.258) (end 33.528 32.258) (width 0.25) (layer "F.Cu") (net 4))
 (segment (start 33.274 32.258) (end 33.147 32.385) (width 0.25) (layer "F.Cu") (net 4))
 (segment (start 33.528 32.258) (end 33.274 32.258) (width 0.25) (layer "F.Cu") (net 4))
 (segment (start 34.772 25.68) (end 34.772 25.4) (width 0.25) (layer "F.Cu") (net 4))
 (segment (start 35.941 33.69) (end 35.941 32.385) (width 0.25) (layer "F.Cu") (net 4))
 (segment (start 38.481 28.54) (end 38.481 29.21) (width 0.25) (layer "F.Cu") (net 4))
 (segment (start 32.7 32.832) (end 32.7 33.6065) (width 0.25) (layer "F.Cu") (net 4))
 (segment (start 38.481 29.845) (end 36.576 31.75) (width 0.25) (layer "F.Cu") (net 4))
 (segment (start 36.068 32.258) (end 36.576 31.75) (width 0.25) (layer "F.Cu") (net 4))
 (segment (start 36.576 31.75) (end 35.941 32.385) (width 0.25) (layer "F.Cu") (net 4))
 (segment (start 35.814 32.258) (end 36.068 32.258) (width 0.25) (layer "F.Cu") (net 4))
 (segment (start 33.528 32.258) (end 33.528 26.644) (width 0.25) (layer "F.Cu") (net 4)))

